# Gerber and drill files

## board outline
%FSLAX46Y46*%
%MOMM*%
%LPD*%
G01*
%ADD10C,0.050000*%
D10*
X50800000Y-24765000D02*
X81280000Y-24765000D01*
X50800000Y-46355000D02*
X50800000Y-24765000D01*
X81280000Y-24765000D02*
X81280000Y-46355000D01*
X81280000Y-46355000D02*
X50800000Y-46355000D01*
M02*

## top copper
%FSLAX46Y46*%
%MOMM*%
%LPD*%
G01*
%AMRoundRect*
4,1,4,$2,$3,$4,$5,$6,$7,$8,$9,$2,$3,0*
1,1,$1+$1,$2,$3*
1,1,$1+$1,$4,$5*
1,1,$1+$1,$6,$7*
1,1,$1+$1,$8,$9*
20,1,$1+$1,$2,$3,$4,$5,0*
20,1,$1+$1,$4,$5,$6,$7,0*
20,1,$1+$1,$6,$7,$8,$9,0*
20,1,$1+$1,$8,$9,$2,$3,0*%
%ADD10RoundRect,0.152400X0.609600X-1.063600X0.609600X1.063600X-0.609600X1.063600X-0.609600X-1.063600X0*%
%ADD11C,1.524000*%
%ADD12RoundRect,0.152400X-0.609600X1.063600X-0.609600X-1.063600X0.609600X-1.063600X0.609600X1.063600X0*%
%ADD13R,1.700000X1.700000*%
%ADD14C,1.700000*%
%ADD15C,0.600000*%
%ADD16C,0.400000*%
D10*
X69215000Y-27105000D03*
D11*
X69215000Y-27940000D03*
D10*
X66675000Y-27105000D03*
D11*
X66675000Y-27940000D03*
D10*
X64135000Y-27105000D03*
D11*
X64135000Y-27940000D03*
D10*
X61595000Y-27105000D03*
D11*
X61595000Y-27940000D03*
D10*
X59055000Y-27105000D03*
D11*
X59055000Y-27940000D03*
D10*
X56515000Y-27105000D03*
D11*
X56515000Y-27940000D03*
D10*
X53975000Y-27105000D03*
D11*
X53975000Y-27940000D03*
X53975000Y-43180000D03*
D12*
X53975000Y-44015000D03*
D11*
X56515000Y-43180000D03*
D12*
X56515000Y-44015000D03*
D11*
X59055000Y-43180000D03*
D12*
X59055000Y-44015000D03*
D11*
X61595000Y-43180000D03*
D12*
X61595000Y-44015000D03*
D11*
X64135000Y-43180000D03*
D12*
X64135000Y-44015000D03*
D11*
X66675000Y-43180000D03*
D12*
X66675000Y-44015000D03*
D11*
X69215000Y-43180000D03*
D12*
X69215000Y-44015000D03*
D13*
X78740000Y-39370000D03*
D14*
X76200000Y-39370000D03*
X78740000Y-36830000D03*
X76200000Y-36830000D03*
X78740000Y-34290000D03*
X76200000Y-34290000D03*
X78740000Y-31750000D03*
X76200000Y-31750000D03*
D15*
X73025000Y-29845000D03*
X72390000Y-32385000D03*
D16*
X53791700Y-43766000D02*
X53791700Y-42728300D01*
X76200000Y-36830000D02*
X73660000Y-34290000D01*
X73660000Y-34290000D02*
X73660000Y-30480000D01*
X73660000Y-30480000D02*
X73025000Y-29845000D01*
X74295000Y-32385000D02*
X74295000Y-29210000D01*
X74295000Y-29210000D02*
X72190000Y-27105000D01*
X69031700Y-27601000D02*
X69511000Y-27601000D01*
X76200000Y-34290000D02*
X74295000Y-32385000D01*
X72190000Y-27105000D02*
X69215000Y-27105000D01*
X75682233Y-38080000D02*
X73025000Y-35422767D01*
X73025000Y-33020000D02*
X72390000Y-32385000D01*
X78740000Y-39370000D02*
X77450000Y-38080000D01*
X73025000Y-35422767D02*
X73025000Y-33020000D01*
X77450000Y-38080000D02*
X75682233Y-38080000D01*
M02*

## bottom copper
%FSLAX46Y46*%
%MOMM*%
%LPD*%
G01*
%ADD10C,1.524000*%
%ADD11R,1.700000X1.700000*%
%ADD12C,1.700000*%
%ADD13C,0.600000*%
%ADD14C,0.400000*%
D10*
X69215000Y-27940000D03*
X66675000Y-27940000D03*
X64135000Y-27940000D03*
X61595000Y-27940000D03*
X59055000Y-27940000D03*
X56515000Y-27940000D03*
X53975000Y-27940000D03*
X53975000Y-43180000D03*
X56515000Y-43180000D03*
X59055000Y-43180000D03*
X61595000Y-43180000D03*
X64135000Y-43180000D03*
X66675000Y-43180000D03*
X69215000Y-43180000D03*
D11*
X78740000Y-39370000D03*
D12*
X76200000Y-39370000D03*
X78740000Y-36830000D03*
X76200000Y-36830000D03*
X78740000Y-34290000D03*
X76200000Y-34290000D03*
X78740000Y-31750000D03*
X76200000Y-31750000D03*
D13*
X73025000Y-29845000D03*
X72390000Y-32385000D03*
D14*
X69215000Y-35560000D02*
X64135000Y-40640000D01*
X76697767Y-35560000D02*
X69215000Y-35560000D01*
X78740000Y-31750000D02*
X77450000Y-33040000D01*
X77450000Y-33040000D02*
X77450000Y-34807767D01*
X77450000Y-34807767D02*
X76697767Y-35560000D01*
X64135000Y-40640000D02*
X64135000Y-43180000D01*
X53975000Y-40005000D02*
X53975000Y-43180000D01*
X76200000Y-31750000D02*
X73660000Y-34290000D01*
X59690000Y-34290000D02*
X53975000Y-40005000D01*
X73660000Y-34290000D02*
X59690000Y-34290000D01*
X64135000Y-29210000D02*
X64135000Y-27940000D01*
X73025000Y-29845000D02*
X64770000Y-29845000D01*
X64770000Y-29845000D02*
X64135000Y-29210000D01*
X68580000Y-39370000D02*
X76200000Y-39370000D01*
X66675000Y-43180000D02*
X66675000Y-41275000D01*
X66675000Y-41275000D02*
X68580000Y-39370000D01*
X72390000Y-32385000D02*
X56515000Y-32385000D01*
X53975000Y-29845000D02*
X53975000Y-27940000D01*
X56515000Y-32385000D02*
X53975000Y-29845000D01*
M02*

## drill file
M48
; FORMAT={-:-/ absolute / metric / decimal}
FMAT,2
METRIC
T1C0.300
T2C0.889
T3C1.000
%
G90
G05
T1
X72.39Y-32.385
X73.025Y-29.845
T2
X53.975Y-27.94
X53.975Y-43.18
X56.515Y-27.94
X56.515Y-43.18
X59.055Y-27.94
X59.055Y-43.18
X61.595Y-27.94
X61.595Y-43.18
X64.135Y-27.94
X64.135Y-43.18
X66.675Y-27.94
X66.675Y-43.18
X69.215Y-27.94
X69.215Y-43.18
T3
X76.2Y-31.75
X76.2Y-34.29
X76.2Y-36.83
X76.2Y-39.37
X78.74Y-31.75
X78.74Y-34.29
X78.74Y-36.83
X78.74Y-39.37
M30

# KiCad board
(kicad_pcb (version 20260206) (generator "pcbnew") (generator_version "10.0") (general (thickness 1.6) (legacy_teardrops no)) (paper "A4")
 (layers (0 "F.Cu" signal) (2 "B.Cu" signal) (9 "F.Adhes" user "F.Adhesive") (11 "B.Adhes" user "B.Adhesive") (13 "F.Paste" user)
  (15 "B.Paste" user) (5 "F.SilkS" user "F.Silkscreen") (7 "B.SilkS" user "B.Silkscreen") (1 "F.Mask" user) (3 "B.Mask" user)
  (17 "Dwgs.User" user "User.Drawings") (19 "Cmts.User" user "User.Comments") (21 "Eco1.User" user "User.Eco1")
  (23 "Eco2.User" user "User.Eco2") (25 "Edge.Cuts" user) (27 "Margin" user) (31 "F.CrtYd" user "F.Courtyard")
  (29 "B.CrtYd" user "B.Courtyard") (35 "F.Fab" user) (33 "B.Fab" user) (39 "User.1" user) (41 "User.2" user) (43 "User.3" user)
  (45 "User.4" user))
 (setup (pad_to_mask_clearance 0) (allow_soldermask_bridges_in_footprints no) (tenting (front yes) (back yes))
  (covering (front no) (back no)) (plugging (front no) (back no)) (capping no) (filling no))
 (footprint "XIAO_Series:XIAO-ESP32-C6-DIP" (layer "F.Cu") (at 61.595 35.56)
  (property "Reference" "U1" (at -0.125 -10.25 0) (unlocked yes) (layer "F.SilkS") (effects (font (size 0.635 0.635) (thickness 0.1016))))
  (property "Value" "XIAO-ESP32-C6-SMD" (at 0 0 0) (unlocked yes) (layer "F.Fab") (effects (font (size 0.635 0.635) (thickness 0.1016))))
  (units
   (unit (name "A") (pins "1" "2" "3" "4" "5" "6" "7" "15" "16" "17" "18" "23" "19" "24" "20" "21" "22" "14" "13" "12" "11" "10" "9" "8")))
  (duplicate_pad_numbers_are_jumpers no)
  (pad "1" smd roundrect (at 7.62 -8.455 90) (size 2.432 1.524) (layers "F.Cu" "F.Mask") (roundrect_rratio 0.1) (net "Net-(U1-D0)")
   (thermal_bridge_angle 45))
  (pad "1" thru_hole circle (at 7.62 -7.62 90) (size 1.524 1.524) (drill 0.889) (layers "*.Cu" "*.Mask") (remove_unused_layers no)
   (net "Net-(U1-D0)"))
  (pad "2" smd roundrect (at 5.08 -8.455 90) (size 2.432 1.524) (layers "F.Cu" "F.Mask") (roundrect_rratio 0.1)
   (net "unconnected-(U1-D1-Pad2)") (thermal_bridge_angle 45))
  (pad "2" thru_hole circle (at 5.08 -7.62 90) (size 1.524 1.524) (drill 0.889) (layers "*.Cu" "*.Mask") (remove_unused_layers no)
   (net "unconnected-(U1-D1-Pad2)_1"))
  (pad "3" smd roundrect (at 2.54 -8.455 90) (size 2.432 1.524) (layers "F.Cu" "F.Mask") (roundrect_rratio 0.1) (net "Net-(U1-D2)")
   (thermal_bridge_angle 45))
  (pad "3" thru_hole circle (at 2.54 -7.62 90) (size 1.524 1.524) (drill 0.889) (layers "*.Cu" "*.Mask") (remove_unused_layers no)
   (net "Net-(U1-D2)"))
  (pad "4" smd roundrect (at 0 -8.455 90) (size 2.432 1.524) (layers "F.Cu" "F.Mask") (roundrect_rratio 0.1)
   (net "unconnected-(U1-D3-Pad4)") (thermal_bridge_angle 45))
  (pad "4" thru_hole circle (at 0 -7.62 90) (size 1.524 1.524) (drill 0.889) (layers "*.Cu" "*.Mask") (remove_unused_layers no)
   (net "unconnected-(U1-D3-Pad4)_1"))
  (pad "5" smd roundrect (at -2.54 -8.455 90) (size 2.432 1.524) (layers "F.Cu" "F.Mask") (roundrect_rratio 0.1)
   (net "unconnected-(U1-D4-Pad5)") (thermal_bridge_angle 45))
  (pad "5" thru_hole circle (at -2.54 -7.62 90) (size 1.524 1.524) (drill 0.889) (layers "*.Cu" "*.Mask") (remove_unused_layers no)
   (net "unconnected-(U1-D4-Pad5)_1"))
  (pad "6" smd roundrect (at -5.08 -8.455 90) (size 2.432 1.524) (layers "F.Cu" "F.Mask") (roundrect_rratio 0.1)
   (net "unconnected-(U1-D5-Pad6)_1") (thermal_bridge_angle 45))
  (pad "6" thru_hole circle (at -5.08 -7.62 90) (size 1.524 1.524) (drill 0.889) (layers "*.Cu" "*.Mask") (remove_unused_layers no)
   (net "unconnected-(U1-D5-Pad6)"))
  (pad "7" smd roundrect (at -7.62 -8.455 90) (size 2.432 1.524) (layers "F.Cu" "F.Mask") (roundrect_rratio 0.1) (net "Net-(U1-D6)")
   (thermal_bridge_angle 45))
  (pad "7" thru_hole circle (at -7.62 -7.62 90) (size 1.524 1.524) (drill 0.889) (layers "*.Cu" "*.Mask") (remove_unused_layers no)
   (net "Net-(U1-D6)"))
  (pad "8" thru_hole circle (at -7.62 7.62 270) (size 1.524 1.524) (drill 0.889) (layers "*.Cu" "*.Mask") (remove_unused_layers no)
   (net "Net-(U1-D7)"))
  (pad "8" smd roundrect (at -7.62 8.455 270) (size 2.432 1.524) (layers "F.Cu" "F.Mask") (roundrect_rratio 0.1) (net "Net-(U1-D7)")
   (thermal_bridge_angle 45))
  (pad "9" thru_hole circle (at -5.08 7.62 270) (size 1.524 1.524) (drill 0.889) (layers "*.Cu" "*.Mask") (remove_unused_layers no)
   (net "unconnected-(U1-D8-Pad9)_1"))
  (pad "9" smd roundrect (at -5.08 8.455 270) (size 2.432 1.524) (layers "F.Cu" "F.Mask") (roundrect_rratio 0.1)
   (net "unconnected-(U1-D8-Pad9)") (thermal_bridge_angle 45))
  (pad "10" thru_hole circle (at -2.54 7.62 270) (size 1.524 1.524) (drill 0.889) (layers "*.Cu" "*.Mask") (remove_unused_layers no)
   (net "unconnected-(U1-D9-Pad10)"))
  (pad "10" smd roundrect (at -2.54 8.455 270) (size 2.432 1.524) (layers "F.Cu" "F.Mask") (roundrect_rratio 0.1)
   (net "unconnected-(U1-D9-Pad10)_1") (thermal_bridge_angle 45))
  (pad "11" thru_hole circle (at 0 7.62 270) (size 1.524 1.524) (drill 0.889) (layers "*.Cu" "*.Mask") (remove_unused_layers no)
   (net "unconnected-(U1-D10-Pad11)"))
  (pad "11" smd roundrect (at 0 8.455 270) (size 2.432 1.524) (layers "F.Cu" "F.Mask") (roundrect_rratio 0.1)
   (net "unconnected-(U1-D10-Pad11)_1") (thermal_bridge_angle 45))
  (pad "12" thru_hole circle (at 2.54 7.62 270) (size 1.524 1.524) (drill 0.889) (layers "*.Cu" "*.Mask") (remove_unused_layers no)
   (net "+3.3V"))
  (pad "12" smd roundrect (at 2.54 8.455 270) (size 2.432 1.524) (layers "F.Cu" "F.Mask") (roundrect_rratio 0.1) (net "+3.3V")
   (thermal_bridge_angle 45))
  (pad "13" thru_hole circle (at 5.08 7.62 270) (size 1.524 1.524) (drill 0.889) (layers "*.Cu" "*.Mask") (remove_unused_layers no)
   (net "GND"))
  (pad "13" smd roundrect (at 5.08 8.455 270) (size 2.432 1.524) (layers "F.Cu" "F.Mask") (roundrect_rratio 0.1) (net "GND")
   (thermal_bridge_angle 45))
  (pad "14" thru_hole circle (at 7.62 7.62 270) (size 1.524 1.524) (drill 0.889) (layers "*.Cu" "*.Mask") (remove_unused_layers no)
   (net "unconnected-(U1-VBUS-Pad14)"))
  (pad "14" smd roundrect (at 7.62 8.455 270) (size 2.432 1.524) (layers "F.Cu" "F.Mask") (roundrect_rratio 0.1)
   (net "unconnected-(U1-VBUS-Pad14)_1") (thermal_bridge_angle 45)))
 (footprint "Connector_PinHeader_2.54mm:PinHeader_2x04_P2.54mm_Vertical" (layer "F.Cu") (at 78.74 39.37 180)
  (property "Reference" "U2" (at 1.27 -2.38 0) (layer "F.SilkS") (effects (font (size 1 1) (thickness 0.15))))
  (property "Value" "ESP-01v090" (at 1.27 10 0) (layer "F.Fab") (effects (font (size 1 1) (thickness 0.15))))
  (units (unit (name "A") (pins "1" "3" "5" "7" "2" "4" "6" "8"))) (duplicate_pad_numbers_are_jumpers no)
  (pad "1" thru_hole rect (at 0 0 180) (size 1.7 1.7) (drill 1) (layers "*.Cu" "*.Mask") (remove_unused_layers no) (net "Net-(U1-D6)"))
  (pad "2" thru_hole circle (at 2.54 0 180) (size 1.7 1.7) (drill 1) (layers "*.Cu" "*.Mask") (remove_unused_layers no) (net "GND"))
  (pad "3" thru_hole circle (at 0 2.54 180) (size 1.7 1.7) (drill 1) (layers "*.Cu" "*.Mask") (remove_unused_layers no)
   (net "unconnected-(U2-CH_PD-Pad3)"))
  (pad "4" thru_hole circle (at 2.54 2.54 180) (size 1.7 1.7) (drill 1) (layers "*.Cu" "*.Mask") (remove_unused_layers no)
   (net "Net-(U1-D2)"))
  (pad "5" thru_hole circle (at 0 5.08 180) (size 1.7 1.7) (drill 1) (layers "*.Cu" "*.Mask") (remove_unused_layers no)
   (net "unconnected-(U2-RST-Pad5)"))
  (pad "6" thru_hole circle (at 2.54 5.08 180) (size 1.7 1.7) (drill 1) (layers "*.Cu" "*.Mask") (remove_unused_layers no)
   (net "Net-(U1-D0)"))
  (pad "7" thru_hole circle (at 0 7.62 180) (size 1.7 1.7) (drill 1) (layers "*.Cu" "*.Mask") (remove_unused_layers no) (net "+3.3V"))
  (pad "8" thru_hole circle (at 2.54 7.62 180) (size 1.7 1.7) (drill 1) (layers "*.Cu" "*.Mask") (remove_unused_layers no)
   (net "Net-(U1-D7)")))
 (gr_line (start 50.8 24.765) (end 81.28 24.765) (stroke (width 0.05) (type default)) (layer "Edge.Cuts"))
 (gr_line (start 50.8 46.355) (end 50.8 24.765) (stroke (width 0.05) (type default)) (layer "Edge.Cuts"))
 (gr_line (start 81.28 24.765) (end 81.28 46.355) (stroke (width 0.05) (type default)) (layer "Edge.Cuts"))
 (gr_line (start 81.28 46.355) (end 50.8 46.355) (stroke (width 0.05) (type default)) (layer "Edge.Cuts"))
 (segment (start 69.215 35.56) (end 64.135 40.64) (width 0.4) (layer "B.Cu") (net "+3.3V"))
 (segment (start 76.697767 35.56) (end 69.215 35.56) (width 0.4) (layer "B.Cu") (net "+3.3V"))
 (segment (start 78.74 31.75) (end 77.45 33.04) (width 0.4) (layer "B.Cu") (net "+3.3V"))
 (segment (start 77.45 33.04) (end 77.45 34.807767) (width 0.4) (layer "B.Cu") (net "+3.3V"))
 (segment (start 77.45 34.807767) (end 76.697767 35.56) (width 0.4) (layer "B.Cu") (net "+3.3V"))
 (segment (start 64.135 40.64) (end 64.135 43.18) (width 0.4) (layer "B.Cu") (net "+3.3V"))
 (segment (start 53.7917 43.766) (end 53.7917 42.7283) (width 0.4) (layer "F.Cu") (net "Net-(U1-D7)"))
 (segment (start 53.975 40.005) (end 53.975 43.18) (width 0.4) (layer "B.Cu") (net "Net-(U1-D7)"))
 (segment (start 76.2 31.75) (end 73.66 34.29) (width 0.4) (layer "B.Cu") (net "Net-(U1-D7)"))
 (segment (start 59.69 34.29) (end 53.975 40.005) (width 0.4) (layer "B.Cu") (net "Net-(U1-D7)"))
 (segment (start 73.66 34.29) (end 59.69 34.29) (width 0.4) (layer "B.Cu") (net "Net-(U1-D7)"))
 (segment (start 76.2 36.83) (end 73.66 34.29) (width 0.4) (layer "F.Cu") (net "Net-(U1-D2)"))
 (segment (start 73.66 34.29) (end 73.66 30.48) (width 0.4) (layer "F.Cu") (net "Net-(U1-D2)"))
 (segment (start 73.66 30.48) (end 73.025 29.845) (width 0.4) (layer "F.Cu") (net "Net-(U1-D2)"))
 (via (at 73.025 29.845) (size 0.6) (drill 0.3) (layers "F.Cu" "B.Cu") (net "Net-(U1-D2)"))
 (segment (start 64.135 29.21) (end 64.135 27.94) (width 0.4) (layer "B.Cu") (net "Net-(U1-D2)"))
 (segment (start 73.025 29.845) (end 64.77 29.845) (width 0.4) (layer "B.Cu") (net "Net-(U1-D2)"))
 (segment (start 64.77 29.845) (end 64.135 29.21) (width 0.4) (layer "B.Cu") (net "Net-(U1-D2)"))
 (segment (start 74.295 32.385) (end 74.295 29.21) (width 0.4) (layer "F.Cu") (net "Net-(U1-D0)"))
 (segment (start 74.295 29.21) (end 72.19 27.105) (width 0.4) (layer "F.Cu") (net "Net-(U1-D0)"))
 (segment (start 69.0317 27.601) (end 69.511 27.601) (width 0.4) (layer "F.Cu") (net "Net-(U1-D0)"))
 (segment (start 76.2 34.29) (end 74.295 32.385) (width 0.4) (layer "F.Cu") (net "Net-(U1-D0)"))
 (segment (start 72.19 27.105) (end 69.215 27.105) (width 0.4) (layer "F.Cu") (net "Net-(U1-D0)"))
 (segment (start 68.58 39.37) (end 76.2 39.37) (width 0.4) (layer "B.Cu") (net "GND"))
 (segment (start 66.675 43.18) (end 66.675 41.275) (width 0.4) (layer "B.Cu") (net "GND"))
 (segment (start 66.675 41.275) (end 68.58 39.37) (width 0.4) (layer "B.Cu") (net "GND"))
 (segment (start 75.682233 38.08) (end 73.025 35.422767) (width 0.4) (layer "F.Cu") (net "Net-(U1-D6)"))
 (segment (start 73.025 33.02) (end 72.39 32.385) (width 0.4) (layer "F.Cu") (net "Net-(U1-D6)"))
 (segment (start 78.74 39.37) (end 77.45 38.08) (width 0.4) (layer "F.Cu") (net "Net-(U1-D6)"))
 (segment (start 73.025 35.422767) (end 73.025 33.02) (width 0.4) (layer "F.Cu") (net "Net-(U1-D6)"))
 (segment (start 77.45 38.08) (end 75.682233 38.08) (width 0.4) (layer "F.Cu") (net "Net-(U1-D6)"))
 (via (at 72.39 32.385) (size 0.6) (drill 0.3) (layers "F.Cu" "B.Cu") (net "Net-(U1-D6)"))
 (segment (start 72.39 32.385) (end 56.515 32.385) (width 0.4) (layer "B.Cu") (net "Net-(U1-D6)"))
 (segment (start 53.975 29.845) (end 53.975 27.94) (width 0.4) (layer "B.Cu") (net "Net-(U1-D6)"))
 (segment (start 56.515 32.385) (end 53.975 29.845) (width 0.4) (layer "B.Cu") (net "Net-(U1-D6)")))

